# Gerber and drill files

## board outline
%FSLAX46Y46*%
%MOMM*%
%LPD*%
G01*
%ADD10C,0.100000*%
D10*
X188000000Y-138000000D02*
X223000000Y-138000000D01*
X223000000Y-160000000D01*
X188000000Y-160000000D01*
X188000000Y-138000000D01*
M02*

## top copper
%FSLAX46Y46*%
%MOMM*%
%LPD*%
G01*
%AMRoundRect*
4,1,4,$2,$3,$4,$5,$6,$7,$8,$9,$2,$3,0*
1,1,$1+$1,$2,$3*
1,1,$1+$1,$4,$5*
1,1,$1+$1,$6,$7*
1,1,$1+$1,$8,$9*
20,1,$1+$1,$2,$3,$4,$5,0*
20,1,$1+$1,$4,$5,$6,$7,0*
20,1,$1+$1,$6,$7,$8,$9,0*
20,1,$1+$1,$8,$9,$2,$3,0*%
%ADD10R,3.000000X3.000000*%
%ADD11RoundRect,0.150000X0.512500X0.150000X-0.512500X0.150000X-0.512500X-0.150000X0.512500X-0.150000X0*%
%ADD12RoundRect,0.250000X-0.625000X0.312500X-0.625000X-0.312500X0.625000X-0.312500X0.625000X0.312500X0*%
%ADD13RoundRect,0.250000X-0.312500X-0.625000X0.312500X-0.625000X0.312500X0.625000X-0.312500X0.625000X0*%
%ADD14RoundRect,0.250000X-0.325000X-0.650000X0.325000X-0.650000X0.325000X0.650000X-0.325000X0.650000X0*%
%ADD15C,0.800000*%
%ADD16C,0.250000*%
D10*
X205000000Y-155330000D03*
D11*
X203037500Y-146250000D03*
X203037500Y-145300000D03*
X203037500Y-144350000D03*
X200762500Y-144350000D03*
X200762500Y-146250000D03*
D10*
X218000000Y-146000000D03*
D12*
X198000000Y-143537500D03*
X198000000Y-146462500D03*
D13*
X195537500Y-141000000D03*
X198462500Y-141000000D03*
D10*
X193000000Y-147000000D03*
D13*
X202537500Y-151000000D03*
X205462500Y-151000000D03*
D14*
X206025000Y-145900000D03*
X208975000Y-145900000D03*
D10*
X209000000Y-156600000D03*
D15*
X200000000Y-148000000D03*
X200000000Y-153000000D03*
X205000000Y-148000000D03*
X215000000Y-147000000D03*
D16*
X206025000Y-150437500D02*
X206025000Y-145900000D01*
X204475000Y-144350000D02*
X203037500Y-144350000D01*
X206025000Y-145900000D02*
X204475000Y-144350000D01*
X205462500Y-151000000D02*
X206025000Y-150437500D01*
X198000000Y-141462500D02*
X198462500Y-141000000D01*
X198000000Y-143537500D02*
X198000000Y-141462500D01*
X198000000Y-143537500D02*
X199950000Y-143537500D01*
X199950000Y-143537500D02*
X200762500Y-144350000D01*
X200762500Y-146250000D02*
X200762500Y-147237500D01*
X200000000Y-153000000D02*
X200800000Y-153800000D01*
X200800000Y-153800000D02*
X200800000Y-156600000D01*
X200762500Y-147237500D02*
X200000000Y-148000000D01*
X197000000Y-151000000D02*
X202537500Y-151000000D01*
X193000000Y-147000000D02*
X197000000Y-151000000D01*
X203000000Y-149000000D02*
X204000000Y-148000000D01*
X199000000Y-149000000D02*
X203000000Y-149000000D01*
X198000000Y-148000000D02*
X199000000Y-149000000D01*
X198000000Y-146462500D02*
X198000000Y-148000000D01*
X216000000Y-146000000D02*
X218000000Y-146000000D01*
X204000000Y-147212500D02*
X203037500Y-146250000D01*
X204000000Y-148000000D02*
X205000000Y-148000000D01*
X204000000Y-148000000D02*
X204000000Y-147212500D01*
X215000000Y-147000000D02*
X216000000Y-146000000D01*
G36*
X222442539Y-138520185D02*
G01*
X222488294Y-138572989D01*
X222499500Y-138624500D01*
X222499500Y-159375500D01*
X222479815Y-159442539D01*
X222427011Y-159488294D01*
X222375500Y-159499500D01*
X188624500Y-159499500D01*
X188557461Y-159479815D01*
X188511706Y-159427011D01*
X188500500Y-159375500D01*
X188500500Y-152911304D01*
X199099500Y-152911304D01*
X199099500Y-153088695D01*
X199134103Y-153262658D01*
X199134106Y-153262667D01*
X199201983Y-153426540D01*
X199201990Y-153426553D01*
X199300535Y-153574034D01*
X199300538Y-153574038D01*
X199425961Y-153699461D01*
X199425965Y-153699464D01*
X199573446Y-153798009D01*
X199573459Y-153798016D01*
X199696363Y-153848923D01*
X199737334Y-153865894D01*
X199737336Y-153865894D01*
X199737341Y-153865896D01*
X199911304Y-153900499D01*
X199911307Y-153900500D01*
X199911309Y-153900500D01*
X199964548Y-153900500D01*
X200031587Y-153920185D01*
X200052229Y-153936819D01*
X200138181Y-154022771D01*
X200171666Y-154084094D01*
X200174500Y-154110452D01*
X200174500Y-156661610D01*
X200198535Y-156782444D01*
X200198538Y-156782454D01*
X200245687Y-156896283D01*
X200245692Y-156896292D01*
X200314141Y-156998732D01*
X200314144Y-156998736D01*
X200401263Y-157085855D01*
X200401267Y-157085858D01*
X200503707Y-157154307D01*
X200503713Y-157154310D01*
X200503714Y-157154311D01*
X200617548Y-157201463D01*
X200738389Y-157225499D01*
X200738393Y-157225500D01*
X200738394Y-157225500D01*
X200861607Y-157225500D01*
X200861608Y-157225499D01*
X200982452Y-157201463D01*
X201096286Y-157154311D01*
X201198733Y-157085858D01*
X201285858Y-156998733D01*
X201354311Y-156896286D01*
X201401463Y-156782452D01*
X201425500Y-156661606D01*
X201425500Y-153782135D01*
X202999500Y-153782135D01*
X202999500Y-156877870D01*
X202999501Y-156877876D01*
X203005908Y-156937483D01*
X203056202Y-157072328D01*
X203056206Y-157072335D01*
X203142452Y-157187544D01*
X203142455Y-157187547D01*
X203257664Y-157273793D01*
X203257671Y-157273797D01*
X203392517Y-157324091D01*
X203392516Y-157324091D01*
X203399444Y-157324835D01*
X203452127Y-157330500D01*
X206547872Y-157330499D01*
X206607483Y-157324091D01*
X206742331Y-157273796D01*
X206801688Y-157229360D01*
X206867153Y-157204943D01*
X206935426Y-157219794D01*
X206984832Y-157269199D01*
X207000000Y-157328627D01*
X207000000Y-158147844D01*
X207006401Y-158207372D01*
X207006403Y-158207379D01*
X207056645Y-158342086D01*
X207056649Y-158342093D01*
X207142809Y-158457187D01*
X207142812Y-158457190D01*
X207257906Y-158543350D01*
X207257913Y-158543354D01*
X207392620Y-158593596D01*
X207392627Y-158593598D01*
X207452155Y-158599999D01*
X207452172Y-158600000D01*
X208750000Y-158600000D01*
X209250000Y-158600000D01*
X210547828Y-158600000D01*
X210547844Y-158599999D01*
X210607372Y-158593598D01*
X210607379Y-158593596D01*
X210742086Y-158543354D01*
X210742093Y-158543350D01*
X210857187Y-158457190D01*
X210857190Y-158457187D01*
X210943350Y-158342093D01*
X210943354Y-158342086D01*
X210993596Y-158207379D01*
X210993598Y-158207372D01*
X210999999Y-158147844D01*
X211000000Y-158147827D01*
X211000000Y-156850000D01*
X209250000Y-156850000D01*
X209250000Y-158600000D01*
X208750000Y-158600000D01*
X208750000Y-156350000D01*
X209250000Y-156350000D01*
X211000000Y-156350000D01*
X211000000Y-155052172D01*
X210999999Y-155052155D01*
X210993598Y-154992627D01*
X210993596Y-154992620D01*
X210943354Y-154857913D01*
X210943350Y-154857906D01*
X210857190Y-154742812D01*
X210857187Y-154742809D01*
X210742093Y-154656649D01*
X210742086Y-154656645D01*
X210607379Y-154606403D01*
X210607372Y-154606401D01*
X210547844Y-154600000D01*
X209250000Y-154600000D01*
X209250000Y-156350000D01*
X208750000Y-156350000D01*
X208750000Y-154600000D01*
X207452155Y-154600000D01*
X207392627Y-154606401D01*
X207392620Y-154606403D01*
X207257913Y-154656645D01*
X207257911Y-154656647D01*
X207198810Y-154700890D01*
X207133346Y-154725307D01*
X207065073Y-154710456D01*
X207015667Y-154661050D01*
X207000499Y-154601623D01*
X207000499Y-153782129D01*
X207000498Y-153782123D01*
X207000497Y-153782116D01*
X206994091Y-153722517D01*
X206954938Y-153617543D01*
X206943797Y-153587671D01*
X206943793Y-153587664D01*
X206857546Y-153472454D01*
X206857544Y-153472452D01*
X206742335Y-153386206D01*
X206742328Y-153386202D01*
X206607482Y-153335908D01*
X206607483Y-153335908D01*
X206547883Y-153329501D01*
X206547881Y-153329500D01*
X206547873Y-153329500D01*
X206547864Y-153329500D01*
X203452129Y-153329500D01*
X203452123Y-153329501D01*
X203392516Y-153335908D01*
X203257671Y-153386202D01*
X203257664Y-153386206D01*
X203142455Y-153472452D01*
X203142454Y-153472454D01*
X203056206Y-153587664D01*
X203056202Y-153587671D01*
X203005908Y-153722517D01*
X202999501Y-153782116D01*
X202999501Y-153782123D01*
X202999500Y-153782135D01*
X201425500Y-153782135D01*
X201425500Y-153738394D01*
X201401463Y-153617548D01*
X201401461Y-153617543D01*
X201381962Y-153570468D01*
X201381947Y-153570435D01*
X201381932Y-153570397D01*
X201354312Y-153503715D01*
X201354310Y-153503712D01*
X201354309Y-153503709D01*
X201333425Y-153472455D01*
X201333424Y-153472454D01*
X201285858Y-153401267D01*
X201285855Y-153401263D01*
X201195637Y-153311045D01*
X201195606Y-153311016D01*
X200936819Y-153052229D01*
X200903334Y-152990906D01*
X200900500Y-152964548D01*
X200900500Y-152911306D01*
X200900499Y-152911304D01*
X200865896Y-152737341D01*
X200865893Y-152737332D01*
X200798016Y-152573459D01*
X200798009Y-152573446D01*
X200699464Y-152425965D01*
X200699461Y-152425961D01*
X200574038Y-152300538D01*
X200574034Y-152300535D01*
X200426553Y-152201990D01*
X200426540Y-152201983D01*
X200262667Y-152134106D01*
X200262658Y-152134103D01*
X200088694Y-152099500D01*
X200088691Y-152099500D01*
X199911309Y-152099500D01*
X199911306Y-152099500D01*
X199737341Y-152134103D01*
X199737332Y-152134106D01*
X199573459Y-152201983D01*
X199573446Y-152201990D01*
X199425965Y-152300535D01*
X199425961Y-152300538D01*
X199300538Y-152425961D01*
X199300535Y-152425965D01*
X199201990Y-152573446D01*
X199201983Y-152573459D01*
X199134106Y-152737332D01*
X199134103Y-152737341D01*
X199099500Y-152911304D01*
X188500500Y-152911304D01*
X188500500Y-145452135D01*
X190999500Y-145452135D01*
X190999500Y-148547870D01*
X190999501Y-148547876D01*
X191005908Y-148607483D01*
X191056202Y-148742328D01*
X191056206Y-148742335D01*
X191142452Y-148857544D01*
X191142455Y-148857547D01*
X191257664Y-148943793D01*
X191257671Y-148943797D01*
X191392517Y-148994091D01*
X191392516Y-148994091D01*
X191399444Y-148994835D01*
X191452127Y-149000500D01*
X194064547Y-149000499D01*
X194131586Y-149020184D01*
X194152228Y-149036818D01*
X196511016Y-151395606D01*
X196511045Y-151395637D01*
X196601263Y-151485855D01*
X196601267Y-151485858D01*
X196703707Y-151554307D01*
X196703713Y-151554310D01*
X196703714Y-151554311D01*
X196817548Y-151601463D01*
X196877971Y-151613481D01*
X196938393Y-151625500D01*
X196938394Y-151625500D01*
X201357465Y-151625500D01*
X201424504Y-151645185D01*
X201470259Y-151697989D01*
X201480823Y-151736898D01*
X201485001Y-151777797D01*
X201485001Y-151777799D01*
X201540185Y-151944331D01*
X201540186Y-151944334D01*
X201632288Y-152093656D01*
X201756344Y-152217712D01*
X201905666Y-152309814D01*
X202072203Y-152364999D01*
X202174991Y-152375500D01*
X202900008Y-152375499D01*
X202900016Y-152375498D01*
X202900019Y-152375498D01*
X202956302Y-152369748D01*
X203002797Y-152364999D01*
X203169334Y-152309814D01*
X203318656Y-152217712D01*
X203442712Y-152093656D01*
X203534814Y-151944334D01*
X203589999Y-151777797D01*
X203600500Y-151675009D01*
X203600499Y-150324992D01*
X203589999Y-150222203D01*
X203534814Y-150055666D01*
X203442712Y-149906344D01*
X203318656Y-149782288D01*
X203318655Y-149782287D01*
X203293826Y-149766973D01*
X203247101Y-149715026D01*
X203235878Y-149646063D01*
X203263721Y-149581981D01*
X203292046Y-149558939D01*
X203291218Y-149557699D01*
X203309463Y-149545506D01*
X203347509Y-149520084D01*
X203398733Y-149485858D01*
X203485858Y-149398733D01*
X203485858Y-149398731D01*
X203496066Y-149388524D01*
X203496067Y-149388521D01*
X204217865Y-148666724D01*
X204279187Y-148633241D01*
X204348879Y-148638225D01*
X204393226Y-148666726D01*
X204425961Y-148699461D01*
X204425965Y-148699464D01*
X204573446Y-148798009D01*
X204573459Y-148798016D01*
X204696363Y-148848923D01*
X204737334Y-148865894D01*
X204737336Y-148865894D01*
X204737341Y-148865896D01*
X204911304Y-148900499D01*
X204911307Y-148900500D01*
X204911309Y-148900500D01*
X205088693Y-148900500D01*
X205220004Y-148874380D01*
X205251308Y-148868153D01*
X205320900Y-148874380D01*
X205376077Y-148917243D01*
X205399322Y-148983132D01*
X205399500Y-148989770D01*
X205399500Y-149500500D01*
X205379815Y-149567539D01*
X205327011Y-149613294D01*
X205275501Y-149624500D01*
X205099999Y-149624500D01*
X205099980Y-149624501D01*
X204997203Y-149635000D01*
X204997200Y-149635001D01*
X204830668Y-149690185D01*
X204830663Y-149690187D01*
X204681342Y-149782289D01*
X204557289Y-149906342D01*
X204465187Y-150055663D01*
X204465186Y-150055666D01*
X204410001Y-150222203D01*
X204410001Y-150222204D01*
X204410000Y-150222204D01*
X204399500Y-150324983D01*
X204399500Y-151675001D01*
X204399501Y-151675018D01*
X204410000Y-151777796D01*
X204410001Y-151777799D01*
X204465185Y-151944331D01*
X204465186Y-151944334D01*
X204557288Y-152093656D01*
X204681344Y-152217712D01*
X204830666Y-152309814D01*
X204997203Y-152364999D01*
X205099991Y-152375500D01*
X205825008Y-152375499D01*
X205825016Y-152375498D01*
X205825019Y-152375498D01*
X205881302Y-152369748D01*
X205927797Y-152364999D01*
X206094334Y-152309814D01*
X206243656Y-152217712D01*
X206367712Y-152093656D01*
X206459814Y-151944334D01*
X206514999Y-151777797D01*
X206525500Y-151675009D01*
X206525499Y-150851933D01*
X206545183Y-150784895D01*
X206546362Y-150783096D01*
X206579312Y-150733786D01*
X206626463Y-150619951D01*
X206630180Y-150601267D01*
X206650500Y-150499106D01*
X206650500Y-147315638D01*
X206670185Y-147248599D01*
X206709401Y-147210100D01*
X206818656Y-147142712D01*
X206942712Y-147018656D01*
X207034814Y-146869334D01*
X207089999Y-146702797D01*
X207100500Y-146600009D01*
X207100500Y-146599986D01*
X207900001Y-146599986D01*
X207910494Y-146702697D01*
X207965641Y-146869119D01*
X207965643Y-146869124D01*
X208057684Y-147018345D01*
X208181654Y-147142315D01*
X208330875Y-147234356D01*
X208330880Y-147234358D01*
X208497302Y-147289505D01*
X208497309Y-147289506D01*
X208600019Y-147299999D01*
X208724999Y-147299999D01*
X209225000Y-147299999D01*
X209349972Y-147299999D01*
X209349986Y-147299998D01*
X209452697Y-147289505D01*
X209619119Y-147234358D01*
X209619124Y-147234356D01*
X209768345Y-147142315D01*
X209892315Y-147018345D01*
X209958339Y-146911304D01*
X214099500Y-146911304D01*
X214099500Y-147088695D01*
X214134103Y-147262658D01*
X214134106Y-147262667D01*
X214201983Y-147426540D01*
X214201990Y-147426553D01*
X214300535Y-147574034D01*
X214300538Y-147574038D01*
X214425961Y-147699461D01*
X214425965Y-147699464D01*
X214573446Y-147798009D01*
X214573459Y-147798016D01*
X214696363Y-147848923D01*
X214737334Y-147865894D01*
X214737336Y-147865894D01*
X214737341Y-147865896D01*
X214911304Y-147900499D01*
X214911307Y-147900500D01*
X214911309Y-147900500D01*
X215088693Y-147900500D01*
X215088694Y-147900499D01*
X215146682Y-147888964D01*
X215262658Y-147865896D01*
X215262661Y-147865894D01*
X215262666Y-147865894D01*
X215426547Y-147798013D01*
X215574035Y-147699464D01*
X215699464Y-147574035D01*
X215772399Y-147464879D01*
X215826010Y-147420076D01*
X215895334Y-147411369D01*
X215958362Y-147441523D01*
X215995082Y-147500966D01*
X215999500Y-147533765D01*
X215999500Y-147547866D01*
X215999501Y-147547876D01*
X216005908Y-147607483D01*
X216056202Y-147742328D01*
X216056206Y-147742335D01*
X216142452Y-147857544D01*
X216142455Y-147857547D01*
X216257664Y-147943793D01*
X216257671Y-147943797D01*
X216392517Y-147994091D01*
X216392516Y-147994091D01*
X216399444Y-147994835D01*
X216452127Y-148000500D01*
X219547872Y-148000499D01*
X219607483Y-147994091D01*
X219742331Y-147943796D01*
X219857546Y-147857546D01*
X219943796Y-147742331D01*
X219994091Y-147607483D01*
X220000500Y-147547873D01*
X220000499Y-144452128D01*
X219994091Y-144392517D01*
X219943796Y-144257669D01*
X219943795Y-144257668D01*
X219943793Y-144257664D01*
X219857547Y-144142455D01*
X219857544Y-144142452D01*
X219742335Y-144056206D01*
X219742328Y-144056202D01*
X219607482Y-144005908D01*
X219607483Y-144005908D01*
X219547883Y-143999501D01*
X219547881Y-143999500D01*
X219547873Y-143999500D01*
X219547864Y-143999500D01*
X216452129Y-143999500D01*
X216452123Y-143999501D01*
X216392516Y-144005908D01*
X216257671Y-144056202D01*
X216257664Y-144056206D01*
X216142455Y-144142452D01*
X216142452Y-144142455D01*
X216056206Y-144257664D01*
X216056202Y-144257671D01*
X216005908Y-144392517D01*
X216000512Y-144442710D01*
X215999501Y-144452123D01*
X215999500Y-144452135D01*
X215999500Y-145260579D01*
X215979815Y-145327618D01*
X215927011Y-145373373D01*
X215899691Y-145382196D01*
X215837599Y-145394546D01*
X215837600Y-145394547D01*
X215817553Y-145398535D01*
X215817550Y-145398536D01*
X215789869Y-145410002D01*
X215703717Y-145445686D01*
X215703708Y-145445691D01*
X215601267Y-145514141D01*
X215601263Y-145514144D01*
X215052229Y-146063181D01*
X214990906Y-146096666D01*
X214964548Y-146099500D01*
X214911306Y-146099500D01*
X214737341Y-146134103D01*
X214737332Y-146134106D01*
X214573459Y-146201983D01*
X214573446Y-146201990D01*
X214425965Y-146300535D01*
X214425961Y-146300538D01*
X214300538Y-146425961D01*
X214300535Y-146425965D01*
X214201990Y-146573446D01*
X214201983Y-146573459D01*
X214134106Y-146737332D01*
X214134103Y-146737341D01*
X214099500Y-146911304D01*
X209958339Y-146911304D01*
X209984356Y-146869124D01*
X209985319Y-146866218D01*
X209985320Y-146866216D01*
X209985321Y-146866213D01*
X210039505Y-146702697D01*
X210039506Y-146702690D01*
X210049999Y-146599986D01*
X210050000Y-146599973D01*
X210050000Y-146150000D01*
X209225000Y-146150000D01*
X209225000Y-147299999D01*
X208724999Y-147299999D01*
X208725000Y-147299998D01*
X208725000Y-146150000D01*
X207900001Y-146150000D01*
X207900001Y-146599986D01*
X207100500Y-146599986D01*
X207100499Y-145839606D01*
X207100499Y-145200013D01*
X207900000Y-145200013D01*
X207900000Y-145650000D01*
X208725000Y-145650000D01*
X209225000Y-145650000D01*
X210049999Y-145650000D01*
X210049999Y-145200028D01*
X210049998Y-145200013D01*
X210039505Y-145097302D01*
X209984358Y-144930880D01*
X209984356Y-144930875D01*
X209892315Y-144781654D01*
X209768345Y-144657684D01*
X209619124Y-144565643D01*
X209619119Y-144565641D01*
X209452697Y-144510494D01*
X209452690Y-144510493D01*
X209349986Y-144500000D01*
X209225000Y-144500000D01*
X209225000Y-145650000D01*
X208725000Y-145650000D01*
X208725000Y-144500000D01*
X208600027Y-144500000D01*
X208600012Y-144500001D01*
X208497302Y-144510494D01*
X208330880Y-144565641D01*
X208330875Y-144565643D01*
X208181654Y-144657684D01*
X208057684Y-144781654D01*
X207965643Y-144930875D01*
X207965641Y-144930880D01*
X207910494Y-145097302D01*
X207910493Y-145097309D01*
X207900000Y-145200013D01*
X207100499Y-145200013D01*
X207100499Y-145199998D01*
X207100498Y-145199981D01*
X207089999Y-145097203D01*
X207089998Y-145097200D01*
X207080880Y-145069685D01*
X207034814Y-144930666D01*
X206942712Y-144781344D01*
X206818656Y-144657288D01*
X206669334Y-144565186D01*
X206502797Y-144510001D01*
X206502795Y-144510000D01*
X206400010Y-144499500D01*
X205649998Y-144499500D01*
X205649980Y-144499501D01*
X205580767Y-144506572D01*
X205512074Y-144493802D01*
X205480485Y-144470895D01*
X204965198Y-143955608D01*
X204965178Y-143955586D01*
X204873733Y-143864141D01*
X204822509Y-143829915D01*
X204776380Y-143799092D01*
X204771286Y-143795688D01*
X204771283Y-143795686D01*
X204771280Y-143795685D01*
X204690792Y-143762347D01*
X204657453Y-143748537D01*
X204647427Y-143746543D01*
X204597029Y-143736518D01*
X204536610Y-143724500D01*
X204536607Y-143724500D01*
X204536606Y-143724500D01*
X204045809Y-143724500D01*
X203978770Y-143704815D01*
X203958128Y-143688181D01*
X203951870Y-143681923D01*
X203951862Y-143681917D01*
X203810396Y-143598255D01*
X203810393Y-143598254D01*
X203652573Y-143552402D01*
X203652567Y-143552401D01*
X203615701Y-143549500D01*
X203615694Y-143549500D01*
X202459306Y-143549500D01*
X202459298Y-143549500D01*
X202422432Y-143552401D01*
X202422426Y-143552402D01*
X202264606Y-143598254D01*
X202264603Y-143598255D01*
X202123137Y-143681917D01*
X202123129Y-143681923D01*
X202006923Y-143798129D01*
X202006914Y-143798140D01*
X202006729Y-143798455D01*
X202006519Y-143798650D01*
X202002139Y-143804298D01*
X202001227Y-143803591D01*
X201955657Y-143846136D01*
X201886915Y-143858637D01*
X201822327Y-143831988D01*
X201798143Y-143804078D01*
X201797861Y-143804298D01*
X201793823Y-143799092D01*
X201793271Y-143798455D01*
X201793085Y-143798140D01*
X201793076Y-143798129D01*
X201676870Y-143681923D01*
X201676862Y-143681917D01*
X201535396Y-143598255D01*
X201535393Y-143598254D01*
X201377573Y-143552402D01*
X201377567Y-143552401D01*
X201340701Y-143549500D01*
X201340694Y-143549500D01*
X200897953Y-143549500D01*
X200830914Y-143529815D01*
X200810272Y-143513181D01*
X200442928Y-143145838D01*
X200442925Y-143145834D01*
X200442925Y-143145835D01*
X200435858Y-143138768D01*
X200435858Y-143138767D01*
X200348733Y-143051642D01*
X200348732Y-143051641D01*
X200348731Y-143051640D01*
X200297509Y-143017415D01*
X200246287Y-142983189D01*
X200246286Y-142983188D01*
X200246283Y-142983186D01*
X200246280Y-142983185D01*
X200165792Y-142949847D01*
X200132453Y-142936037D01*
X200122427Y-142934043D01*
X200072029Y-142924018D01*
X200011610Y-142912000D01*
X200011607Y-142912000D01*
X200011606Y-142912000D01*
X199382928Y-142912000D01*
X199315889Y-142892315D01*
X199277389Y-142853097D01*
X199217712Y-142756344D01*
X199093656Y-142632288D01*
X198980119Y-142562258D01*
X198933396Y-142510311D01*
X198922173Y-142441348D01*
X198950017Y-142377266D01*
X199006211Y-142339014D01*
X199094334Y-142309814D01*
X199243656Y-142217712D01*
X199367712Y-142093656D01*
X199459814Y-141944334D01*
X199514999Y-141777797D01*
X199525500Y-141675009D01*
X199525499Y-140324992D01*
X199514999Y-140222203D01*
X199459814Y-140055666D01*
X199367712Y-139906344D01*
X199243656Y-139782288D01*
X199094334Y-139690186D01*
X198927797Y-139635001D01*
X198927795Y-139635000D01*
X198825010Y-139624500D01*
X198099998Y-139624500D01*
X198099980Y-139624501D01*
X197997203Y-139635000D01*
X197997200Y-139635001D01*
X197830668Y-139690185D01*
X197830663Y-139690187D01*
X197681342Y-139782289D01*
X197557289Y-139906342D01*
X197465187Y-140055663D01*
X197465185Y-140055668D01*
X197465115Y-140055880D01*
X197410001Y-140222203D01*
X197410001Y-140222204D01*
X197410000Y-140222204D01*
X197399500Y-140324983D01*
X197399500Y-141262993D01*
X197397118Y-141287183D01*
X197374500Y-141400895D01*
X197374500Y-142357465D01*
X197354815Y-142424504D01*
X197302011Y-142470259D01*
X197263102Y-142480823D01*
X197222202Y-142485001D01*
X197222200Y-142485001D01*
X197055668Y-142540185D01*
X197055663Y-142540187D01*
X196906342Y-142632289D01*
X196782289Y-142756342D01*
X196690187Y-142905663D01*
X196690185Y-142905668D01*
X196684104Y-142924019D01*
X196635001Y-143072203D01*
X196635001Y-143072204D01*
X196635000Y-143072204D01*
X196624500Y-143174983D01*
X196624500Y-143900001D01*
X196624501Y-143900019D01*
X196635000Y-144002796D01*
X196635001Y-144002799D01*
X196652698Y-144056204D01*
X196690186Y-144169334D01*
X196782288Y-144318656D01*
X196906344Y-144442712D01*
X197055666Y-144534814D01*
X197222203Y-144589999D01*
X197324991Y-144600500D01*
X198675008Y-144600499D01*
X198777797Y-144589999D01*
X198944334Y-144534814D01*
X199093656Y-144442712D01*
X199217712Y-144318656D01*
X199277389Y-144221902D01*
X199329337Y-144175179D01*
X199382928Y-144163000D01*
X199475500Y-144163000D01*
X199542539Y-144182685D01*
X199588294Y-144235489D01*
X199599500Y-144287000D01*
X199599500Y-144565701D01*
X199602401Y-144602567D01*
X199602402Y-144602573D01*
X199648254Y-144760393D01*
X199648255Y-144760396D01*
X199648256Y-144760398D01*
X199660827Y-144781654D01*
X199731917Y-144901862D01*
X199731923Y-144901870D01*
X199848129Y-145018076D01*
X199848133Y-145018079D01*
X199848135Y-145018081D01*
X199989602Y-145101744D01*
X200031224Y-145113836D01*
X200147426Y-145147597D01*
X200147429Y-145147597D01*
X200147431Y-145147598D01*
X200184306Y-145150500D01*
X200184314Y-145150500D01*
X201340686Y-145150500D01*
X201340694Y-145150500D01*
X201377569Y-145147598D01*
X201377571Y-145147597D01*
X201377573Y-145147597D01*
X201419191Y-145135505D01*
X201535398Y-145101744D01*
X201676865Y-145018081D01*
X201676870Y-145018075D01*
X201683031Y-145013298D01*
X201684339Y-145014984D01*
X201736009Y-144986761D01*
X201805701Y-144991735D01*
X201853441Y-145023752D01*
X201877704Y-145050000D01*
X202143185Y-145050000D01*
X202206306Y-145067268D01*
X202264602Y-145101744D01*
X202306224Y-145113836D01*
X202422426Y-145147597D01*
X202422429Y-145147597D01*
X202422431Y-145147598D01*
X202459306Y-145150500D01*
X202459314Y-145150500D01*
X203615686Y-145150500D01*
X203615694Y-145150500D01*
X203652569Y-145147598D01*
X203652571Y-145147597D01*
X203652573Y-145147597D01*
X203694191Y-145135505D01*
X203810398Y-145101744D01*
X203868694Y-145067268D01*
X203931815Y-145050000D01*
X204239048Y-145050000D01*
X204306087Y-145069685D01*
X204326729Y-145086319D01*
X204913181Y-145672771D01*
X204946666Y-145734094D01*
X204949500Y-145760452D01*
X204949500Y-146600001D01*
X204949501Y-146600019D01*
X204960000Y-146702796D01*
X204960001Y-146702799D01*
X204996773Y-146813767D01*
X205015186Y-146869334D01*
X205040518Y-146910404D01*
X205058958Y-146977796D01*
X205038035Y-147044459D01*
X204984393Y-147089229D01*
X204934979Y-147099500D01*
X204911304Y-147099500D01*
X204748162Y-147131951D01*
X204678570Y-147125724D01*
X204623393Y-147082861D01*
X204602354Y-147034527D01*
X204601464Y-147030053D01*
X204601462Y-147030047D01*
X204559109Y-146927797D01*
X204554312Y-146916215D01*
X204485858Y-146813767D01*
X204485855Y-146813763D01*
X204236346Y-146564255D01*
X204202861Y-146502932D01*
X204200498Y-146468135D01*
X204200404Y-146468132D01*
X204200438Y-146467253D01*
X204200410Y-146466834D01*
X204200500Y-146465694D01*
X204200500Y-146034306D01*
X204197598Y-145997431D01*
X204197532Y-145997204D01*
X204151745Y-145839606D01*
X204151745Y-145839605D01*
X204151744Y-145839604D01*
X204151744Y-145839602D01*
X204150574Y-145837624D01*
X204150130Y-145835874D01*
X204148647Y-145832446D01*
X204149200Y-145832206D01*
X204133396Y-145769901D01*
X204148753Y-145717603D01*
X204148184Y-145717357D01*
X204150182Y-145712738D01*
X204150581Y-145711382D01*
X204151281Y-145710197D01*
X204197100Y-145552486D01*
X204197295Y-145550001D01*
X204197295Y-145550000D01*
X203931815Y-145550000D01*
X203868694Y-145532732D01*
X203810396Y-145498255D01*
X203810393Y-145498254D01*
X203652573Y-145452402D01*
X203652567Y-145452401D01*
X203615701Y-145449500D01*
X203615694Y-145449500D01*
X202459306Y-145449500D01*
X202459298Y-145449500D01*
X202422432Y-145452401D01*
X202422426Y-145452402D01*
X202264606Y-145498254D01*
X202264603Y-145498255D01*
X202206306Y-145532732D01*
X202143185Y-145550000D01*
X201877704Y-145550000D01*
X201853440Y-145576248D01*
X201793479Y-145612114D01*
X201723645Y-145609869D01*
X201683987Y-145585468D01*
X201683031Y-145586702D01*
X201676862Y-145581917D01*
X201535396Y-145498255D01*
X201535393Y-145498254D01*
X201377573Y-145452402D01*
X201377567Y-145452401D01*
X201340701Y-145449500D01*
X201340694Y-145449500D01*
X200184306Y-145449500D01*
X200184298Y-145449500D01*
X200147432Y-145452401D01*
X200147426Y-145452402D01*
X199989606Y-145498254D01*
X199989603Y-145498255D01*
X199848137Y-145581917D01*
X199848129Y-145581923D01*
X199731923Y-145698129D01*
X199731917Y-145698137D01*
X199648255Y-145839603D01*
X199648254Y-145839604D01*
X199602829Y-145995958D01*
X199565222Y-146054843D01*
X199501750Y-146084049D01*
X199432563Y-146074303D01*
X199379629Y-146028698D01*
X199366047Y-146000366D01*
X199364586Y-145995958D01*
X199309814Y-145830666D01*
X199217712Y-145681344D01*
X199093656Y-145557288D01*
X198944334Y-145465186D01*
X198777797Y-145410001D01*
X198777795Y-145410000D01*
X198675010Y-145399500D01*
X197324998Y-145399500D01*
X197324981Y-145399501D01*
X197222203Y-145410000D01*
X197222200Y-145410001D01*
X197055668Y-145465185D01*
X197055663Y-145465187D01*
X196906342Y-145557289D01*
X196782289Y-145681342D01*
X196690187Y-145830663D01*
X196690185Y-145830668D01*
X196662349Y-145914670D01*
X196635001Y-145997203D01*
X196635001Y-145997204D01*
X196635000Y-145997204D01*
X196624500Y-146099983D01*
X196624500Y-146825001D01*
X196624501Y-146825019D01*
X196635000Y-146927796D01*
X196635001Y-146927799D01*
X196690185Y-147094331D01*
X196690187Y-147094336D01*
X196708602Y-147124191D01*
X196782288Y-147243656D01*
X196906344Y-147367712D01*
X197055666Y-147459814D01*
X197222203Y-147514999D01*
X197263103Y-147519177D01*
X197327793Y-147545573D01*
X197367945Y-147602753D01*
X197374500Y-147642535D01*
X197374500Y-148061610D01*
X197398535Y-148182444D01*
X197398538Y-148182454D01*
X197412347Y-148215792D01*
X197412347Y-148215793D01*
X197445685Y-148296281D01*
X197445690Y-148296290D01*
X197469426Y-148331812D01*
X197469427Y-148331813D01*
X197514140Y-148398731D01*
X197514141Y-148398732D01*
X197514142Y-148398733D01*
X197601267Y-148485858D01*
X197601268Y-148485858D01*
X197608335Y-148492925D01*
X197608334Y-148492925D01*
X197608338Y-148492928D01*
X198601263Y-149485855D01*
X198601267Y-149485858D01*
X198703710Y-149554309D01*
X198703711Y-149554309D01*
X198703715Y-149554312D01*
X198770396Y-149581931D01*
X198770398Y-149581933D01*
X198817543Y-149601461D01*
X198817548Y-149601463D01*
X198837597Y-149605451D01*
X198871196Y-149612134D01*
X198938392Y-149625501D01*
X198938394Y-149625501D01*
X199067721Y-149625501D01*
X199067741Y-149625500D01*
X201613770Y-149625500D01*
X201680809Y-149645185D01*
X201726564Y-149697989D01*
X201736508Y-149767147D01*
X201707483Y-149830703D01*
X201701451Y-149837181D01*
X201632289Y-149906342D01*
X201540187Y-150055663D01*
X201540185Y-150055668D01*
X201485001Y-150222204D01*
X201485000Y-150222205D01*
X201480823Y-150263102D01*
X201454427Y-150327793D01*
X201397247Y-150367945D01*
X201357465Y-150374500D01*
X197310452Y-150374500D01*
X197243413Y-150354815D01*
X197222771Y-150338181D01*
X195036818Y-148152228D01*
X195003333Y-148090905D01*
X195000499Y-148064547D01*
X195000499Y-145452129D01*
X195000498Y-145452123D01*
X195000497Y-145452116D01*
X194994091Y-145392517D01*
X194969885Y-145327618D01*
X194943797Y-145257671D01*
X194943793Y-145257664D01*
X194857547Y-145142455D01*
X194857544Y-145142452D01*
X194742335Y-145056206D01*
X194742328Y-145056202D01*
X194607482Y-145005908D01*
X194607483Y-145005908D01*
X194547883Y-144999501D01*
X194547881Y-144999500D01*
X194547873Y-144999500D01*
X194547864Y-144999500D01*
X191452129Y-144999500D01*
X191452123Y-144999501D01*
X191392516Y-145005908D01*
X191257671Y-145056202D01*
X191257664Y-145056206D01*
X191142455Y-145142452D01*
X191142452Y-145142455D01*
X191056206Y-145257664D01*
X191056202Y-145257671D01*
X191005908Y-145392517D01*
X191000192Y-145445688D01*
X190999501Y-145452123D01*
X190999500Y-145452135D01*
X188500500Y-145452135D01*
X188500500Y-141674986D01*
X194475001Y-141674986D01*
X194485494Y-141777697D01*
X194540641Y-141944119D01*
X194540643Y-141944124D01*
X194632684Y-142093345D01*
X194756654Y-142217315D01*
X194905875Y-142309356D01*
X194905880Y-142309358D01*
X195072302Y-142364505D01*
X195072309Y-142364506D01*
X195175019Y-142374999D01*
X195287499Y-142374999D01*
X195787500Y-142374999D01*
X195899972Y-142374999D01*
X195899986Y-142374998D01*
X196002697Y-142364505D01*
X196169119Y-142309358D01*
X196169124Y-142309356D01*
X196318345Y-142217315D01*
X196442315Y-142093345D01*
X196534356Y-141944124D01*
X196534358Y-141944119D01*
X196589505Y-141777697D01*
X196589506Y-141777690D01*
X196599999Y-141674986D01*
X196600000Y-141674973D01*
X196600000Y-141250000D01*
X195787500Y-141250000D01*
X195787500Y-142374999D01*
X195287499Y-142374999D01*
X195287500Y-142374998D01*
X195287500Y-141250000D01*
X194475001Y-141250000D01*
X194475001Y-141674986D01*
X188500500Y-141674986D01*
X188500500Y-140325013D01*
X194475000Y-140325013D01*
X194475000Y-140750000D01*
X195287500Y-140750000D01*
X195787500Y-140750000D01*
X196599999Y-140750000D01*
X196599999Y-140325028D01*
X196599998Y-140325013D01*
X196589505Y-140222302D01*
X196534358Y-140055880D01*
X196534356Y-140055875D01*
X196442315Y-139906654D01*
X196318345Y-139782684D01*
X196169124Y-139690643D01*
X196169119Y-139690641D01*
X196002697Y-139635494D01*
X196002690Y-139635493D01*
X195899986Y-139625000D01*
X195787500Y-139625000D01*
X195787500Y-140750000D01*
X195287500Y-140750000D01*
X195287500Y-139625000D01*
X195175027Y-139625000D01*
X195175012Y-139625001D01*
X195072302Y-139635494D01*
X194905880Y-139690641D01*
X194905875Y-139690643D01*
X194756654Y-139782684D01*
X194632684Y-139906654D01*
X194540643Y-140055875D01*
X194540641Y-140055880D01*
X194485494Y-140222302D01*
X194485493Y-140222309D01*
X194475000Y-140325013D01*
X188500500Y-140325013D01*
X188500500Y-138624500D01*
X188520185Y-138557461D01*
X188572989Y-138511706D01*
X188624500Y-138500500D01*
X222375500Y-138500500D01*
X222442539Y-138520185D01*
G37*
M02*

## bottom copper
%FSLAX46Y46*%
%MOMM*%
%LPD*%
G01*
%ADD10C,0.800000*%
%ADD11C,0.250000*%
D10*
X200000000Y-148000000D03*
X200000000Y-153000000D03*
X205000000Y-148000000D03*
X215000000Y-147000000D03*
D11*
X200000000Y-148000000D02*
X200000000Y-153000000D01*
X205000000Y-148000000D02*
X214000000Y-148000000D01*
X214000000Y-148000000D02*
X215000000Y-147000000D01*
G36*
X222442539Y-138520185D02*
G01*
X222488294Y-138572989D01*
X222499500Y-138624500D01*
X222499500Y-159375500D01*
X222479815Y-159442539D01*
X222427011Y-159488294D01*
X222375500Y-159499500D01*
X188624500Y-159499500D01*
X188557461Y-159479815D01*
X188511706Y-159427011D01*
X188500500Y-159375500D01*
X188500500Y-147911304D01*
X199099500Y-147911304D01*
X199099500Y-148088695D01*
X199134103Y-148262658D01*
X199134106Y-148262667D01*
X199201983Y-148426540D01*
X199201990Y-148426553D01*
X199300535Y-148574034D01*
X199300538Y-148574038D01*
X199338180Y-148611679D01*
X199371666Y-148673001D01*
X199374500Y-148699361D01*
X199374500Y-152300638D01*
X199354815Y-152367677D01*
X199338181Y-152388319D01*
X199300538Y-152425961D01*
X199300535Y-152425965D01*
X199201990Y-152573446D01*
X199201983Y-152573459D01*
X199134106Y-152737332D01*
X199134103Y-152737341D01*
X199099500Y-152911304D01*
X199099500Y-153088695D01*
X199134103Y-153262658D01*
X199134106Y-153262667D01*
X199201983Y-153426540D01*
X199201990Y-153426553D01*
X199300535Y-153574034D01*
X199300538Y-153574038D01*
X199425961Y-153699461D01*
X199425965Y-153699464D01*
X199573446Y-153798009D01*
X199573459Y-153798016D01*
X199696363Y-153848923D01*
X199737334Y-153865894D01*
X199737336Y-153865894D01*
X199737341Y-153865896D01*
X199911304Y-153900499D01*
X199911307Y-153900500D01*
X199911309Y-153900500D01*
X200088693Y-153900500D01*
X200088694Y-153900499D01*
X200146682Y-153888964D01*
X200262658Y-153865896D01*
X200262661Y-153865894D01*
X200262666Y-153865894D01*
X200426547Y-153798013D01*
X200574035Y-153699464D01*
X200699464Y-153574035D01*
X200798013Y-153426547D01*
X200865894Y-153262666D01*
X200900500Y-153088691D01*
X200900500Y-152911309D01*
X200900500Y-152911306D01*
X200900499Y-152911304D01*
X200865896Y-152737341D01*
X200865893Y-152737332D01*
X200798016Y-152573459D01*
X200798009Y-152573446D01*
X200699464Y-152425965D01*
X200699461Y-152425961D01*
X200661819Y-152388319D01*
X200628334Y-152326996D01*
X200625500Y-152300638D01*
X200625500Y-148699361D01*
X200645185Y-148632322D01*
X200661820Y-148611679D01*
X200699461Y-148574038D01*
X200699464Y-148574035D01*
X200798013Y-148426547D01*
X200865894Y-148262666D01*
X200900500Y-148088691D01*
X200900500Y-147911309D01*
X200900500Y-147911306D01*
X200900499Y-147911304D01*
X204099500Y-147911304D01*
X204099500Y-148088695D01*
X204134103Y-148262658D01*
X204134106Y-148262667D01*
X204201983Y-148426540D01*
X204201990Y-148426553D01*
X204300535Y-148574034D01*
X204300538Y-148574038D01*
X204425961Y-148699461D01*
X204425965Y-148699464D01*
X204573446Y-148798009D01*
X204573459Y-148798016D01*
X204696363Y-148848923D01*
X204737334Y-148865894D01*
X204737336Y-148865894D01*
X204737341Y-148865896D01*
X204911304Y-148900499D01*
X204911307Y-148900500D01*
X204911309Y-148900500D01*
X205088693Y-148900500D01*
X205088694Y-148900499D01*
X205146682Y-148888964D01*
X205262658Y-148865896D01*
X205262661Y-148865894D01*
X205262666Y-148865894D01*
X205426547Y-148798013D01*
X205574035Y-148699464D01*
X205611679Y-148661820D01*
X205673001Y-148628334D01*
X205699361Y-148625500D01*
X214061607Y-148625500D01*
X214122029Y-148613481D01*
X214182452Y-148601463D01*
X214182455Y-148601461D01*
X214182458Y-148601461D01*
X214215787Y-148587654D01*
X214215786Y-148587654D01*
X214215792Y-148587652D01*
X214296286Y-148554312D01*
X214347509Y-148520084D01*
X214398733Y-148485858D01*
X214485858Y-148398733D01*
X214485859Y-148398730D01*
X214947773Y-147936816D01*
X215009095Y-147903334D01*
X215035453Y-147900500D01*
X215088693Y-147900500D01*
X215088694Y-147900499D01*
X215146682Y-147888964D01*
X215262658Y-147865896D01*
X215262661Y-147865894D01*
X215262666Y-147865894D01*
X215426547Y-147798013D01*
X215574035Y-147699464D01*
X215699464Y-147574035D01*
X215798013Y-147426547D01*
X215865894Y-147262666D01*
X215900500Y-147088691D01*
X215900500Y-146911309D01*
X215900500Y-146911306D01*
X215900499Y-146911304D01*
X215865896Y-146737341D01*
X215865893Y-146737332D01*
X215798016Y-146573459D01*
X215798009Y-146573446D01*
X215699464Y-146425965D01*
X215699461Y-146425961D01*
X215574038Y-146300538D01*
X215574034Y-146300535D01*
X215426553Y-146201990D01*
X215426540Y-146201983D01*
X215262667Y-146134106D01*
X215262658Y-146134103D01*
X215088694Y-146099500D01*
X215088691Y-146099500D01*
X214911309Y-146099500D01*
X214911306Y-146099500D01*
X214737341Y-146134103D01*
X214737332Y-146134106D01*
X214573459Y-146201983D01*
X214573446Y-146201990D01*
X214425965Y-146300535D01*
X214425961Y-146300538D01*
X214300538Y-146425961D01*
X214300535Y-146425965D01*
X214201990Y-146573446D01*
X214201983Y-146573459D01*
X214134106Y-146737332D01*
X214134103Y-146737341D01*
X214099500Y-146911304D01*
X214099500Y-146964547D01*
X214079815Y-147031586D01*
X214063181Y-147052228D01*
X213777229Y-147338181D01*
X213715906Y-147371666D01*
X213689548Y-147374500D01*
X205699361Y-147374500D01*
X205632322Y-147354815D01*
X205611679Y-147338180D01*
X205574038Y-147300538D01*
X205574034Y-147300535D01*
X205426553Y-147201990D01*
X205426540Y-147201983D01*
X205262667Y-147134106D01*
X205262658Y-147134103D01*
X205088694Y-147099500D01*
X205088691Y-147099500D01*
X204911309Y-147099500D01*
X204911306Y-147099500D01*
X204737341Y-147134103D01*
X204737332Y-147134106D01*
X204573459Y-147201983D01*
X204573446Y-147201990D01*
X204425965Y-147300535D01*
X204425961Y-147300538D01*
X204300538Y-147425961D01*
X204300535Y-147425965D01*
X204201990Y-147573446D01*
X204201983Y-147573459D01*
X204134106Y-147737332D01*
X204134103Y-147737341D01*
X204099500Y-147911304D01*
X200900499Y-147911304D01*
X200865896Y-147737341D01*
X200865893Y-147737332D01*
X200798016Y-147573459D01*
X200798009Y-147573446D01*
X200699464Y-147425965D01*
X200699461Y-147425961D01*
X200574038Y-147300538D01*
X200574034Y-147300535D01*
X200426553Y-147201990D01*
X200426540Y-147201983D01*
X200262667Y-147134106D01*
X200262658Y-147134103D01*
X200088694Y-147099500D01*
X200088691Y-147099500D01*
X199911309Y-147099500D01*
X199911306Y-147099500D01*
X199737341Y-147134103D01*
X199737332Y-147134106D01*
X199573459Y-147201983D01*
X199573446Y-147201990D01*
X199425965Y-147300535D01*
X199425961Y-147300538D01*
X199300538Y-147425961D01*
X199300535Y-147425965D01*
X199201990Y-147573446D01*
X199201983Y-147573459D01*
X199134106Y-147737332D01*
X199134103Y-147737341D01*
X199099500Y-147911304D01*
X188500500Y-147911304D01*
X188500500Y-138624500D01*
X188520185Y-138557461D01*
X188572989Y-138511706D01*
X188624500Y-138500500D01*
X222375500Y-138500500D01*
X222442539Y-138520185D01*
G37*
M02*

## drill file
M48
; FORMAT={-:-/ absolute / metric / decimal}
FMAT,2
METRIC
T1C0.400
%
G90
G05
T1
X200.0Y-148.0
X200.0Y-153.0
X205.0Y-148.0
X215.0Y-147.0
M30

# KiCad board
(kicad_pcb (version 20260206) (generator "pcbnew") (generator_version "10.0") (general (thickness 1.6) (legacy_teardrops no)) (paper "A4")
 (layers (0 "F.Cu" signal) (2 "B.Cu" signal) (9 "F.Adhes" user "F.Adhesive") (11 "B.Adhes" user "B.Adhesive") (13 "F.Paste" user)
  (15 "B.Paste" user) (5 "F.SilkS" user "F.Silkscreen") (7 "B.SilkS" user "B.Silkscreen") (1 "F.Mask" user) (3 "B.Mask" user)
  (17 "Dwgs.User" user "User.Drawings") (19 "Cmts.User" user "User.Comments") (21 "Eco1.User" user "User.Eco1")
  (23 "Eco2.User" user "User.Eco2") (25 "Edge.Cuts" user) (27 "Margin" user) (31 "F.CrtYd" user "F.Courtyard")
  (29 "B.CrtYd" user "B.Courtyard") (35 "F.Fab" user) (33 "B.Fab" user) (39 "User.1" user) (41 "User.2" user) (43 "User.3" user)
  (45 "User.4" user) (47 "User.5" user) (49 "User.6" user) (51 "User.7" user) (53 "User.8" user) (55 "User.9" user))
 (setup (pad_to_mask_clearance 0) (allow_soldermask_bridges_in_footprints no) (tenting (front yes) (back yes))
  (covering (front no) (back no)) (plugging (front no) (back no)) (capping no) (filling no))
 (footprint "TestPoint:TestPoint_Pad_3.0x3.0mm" (layer "F.Cu") (at 205 155.33)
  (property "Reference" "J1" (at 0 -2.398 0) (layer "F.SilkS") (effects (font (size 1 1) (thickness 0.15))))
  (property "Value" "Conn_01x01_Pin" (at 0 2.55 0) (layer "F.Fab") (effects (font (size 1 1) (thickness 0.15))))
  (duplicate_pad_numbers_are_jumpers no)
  (pad "1" smd rect (at 0 0) (size 3 3) (layers "F.Cu" "F.Mask") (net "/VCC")))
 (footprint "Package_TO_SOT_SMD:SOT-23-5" (layer "F.Cu") (at 201.9 145.3 180)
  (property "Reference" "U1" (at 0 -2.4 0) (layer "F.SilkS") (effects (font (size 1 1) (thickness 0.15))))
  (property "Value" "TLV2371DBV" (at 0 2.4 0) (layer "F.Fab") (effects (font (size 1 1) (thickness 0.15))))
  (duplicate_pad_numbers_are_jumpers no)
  (pad "1" smd roundrect (at -1.1375 -0.95 180) (size 1.325 0.6) (layers "F.Cu" "F.Mask" "F.Paste") (roundrect_rratio 0.25) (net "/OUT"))
  (pad "2" smd roundrect (at -1.1375 0 180) (size 1.325 0.6) (layers "F.Cu" "F.Mask" "F.Paste") (roundrect_rratio 0.25) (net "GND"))
  (pad "3" smd roundrect (at -1.1375 0.95 180) (size 1.325 0.6) (layers "F.Cu" "F.Mask" "F.Paste") (roundrect_rratio 0.25)
   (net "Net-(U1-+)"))
  (pad "4" smd roundrect (at 1.1375 0.95 180) (size 1.325 0.6) (layers "F.Cu" "F.Mask" "F.Paste") (roundrect_rratio 0.25) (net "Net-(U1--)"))
  (pad "5" smd roundrect (at 1.1375 -0.95 180) (size 1.325 0.6) (layers "F.Cu" "F.Mask" "F.Paste") (roundrect_rratio 0.25) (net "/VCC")))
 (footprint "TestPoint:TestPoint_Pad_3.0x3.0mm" (layer "F.Cu") (at 218 146)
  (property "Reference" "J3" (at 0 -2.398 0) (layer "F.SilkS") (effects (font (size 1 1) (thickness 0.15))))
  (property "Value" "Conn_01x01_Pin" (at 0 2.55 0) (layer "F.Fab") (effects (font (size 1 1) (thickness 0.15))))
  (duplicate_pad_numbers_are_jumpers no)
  (pad "1" smd rect (at 0 0) (size 3 3) (layers "F.Cu" "F.Mask") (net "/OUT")))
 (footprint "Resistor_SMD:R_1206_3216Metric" (layer "F.Cu") (at 198 145 -90)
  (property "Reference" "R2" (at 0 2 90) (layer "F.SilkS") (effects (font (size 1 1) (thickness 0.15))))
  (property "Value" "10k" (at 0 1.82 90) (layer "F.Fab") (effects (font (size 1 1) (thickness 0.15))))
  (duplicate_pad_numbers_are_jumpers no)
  (pad "1" smd roundrect (at -1.4625 0 270) (size 1.125 1.75) (layers "F.Cu" "F.Mask" "F.Paste") (roundrect_rratio 0.222222)
   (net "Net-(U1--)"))
  (pad "2" smd roundrect (at 1.4625 0 270) (size 1.125 1.75) (layers "F.Cu" "F.Mask" "F.Paste") (roundrect_rratio 0.222222) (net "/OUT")))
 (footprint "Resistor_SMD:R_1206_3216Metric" (layer "F.Cu") (at 197 141)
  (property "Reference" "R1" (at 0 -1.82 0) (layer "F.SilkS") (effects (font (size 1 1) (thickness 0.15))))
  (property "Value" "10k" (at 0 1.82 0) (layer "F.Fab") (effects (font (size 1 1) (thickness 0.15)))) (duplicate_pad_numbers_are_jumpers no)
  (pad "1" smd roundrect (at -1.4625 0) (size 1.125 1.75) (layers "F.Cu" "F.Mask" "F.Paste") (roundrect_rratio 0.222222) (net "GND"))
  (pad "2" smd roundrect (at 1.4625 0) (size 1.125 1.75) (layers "F.Cu" "F.Mask" "F.Paste") (roundrect_rratio 0.222222) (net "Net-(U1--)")))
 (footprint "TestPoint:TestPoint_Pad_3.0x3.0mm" (layer "F.Cu") (at 193 147)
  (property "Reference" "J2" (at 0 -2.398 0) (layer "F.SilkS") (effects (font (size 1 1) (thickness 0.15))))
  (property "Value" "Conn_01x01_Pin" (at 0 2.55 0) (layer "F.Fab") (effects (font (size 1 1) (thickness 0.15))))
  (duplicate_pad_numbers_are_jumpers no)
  (pad "1" smd rect (at 0 0) (size 3 3) (layers "F.Cu" "F.Mask") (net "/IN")))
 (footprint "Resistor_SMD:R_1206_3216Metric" (layer "F.Cu") (at 204 151)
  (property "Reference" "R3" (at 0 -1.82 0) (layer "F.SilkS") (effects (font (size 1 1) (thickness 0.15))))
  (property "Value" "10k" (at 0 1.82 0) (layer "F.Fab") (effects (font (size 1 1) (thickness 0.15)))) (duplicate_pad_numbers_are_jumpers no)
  (pad "1" smd roundrect (at -1.4625 0) (size 1.125 1.75) (layers "F.Cu" "F.Mask" "F.Paste") (roundrect_rratio 0.222222) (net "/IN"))
  (pad "2" smd roundrect (at 1.4625 0) (size 1.125 1.75) (layers "F.Cu" "F.Mask" "F.Paste") (roundrect_rratio 0.222222) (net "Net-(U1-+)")))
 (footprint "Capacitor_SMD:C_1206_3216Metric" (layer "F.Cu") (at 207.5 145.9)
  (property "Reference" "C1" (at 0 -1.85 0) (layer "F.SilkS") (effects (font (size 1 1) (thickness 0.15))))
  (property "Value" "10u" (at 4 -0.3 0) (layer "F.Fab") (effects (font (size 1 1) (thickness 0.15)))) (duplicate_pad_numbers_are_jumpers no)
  (pad "1" smd roundrect (at -1.475 0) (size 1.15 1.8) (layers "F.Cu" "F.Mask" "F.Paste") (roundrect_rratio 0.217391) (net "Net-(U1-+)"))
  (pad "2" smd roundrect (at 1.475 0) (size 1.15 1.8) (layers "F.Cu" "F.Mask" "F.Paste") (roundrect_rratio 0.217391) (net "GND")))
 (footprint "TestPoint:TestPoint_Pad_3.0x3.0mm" (layer "F.Cu") (at 209 156.6)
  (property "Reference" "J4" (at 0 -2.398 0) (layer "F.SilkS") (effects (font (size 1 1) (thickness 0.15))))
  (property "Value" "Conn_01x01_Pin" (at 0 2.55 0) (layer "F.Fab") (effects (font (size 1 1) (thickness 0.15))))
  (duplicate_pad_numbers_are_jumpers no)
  (pad "1" smd rect (at 0 0) (size 3 3) (layers "F.Cu" "F.Mask") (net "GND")))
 (gr_rect (start 188 138) (end 223 160) (stroke (width 0.1) (type default)) (fill no) (layer "Edge.Cuts"))
 (segment (start 206.025 150.4375) (end 206.025 145.9) (width 0.25) (layer "F.Cu") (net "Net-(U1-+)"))
 (segment (start 204.475 144.35) (end 203.0375 144.35) (width 0.25) (layer "F.Cu") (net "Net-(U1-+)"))
 (segment (start 206.025 145.9) (end 204.475 144.35) (width 0.25) (layer "F.Cu") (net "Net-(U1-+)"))
 (segment (start 205.4625 151) (end 206.025 150.4375) (width 0.25) (layer "F.Cu") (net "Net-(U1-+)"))
 (segment (start 198 141.4625) (end 198.4625 141) (width 0.25) (layer "F.Cu") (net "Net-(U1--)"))
 (segment (start 198 143.5375) (end 198 141.4625) (width 0.25) (layer "F.Cu") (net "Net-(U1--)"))
 (segment (start 198 143.5375) (end 199.95 143.5375) (width 0.25) (layer "F.Cu") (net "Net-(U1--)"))
 (segment (start 199.95 143.5375) (end 200.7625 144.35) (width 0.25) (layer "F.Cu") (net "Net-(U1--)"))
 (segment (start 200.7625 146.25) (end 200.7625 147.2375) (width 0.25) (layer "F.Cu") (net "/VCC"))
 (segment (start 200 153) (end 200.8 153.8) (width 0.25) (layer "F.Cu") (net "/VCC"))
 (segment (start 200.8 153.8) (end 200.8 156.6) (width 0.25) (layer "F.Cu") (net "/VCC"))
 (segment (start 200.7625 147.2375) (end 200 148) (width 0.25) (layer "F.Cu") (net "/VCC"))
 (via (at 200 148) (size 0.8) (drill 0.4) (layers "F.Cu" "B.Cu") (capping no) (covering (front no) (back no))
  (plugging (front no) (back no)) (filling no) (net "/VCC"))
 (via (at 200 153) (size 0.8) (drill 0.4) (layers "F.Cu" "B.Cu") (capping no) (covering (front no) (back no))
  (plugging (front no) (back no)) (filling no) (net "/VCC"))
 (segment (start 200 148) (end 200 153) (width 0.25) (layer "B.Cu") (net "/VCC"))
 (segment (start 197 151) (end 202.5375 151) (width 0.25) (layer "F.Cu") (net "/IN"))
 (segment (start 193 147) (end 197 151) (width 0.25) (layer "F.Cu") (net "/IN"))
 (segment (start 203 149) (end 204 148) (width 0.25) (layer "F.Cu") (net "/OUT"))
 (segment (start 199 149) (end 203 149) (width 0.25) (layer "F.Cu") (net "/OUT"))
 (segment (start 198 148) (end 199 149) (width 0.25) (layer "F.Cu") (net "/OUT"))
 (segment (start 198 146.4625) (end 198 148) (width 0.25) (layer "F.Cu") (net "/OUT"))
 (segment (start 216 146) (end 218 146) (width 0.25) (layer "F.Cu") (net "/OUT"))
 (segment (start 204 147.2125) (end 203.0375 146.25) (width 0.25) (layer "F.Cu") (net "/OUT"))
 (segment (start 204 148) (end 205 148) (width 0.25) (layer "F.Cu") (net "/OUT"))
 (segment (start 204 148) (end 204 147.2125) (width 0.25) (layer "F.Cu") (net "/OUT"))
 (segment (start 215 147) (end 216 146) (width 0.25) (layer "F.Cu") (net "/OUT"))
 (via (at 205 148) (size 0.8) (drill 0.4) (layers "F.Cu" "B.Cu") (capping no) (covering (front no) (back no))
  (plugging (front no) (back no)) (filling no) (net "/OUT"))
 (via (at 215 147) (size 0.8) (drill 0.4) (layers "F.Cu" "B.Cu") (capping no) (covering (front no) (back no))
  (plugging (front no) (back no)) (filling no) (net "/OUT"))
 (segment (start 205 148) (end 214 148) (width 0.25) (layer "B.Cu") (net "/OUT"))
 (segment (start 214 148) (end 215 147) (width 0.25) (layer "B.Cu") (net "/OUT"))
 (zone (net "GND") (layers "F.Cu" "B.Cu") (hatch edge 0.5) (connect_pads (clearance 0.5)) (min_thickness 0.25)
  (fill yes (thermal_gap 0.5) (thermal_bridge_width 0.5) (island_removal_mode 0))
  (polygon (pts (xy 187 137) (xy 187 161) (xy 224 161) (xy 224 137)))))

